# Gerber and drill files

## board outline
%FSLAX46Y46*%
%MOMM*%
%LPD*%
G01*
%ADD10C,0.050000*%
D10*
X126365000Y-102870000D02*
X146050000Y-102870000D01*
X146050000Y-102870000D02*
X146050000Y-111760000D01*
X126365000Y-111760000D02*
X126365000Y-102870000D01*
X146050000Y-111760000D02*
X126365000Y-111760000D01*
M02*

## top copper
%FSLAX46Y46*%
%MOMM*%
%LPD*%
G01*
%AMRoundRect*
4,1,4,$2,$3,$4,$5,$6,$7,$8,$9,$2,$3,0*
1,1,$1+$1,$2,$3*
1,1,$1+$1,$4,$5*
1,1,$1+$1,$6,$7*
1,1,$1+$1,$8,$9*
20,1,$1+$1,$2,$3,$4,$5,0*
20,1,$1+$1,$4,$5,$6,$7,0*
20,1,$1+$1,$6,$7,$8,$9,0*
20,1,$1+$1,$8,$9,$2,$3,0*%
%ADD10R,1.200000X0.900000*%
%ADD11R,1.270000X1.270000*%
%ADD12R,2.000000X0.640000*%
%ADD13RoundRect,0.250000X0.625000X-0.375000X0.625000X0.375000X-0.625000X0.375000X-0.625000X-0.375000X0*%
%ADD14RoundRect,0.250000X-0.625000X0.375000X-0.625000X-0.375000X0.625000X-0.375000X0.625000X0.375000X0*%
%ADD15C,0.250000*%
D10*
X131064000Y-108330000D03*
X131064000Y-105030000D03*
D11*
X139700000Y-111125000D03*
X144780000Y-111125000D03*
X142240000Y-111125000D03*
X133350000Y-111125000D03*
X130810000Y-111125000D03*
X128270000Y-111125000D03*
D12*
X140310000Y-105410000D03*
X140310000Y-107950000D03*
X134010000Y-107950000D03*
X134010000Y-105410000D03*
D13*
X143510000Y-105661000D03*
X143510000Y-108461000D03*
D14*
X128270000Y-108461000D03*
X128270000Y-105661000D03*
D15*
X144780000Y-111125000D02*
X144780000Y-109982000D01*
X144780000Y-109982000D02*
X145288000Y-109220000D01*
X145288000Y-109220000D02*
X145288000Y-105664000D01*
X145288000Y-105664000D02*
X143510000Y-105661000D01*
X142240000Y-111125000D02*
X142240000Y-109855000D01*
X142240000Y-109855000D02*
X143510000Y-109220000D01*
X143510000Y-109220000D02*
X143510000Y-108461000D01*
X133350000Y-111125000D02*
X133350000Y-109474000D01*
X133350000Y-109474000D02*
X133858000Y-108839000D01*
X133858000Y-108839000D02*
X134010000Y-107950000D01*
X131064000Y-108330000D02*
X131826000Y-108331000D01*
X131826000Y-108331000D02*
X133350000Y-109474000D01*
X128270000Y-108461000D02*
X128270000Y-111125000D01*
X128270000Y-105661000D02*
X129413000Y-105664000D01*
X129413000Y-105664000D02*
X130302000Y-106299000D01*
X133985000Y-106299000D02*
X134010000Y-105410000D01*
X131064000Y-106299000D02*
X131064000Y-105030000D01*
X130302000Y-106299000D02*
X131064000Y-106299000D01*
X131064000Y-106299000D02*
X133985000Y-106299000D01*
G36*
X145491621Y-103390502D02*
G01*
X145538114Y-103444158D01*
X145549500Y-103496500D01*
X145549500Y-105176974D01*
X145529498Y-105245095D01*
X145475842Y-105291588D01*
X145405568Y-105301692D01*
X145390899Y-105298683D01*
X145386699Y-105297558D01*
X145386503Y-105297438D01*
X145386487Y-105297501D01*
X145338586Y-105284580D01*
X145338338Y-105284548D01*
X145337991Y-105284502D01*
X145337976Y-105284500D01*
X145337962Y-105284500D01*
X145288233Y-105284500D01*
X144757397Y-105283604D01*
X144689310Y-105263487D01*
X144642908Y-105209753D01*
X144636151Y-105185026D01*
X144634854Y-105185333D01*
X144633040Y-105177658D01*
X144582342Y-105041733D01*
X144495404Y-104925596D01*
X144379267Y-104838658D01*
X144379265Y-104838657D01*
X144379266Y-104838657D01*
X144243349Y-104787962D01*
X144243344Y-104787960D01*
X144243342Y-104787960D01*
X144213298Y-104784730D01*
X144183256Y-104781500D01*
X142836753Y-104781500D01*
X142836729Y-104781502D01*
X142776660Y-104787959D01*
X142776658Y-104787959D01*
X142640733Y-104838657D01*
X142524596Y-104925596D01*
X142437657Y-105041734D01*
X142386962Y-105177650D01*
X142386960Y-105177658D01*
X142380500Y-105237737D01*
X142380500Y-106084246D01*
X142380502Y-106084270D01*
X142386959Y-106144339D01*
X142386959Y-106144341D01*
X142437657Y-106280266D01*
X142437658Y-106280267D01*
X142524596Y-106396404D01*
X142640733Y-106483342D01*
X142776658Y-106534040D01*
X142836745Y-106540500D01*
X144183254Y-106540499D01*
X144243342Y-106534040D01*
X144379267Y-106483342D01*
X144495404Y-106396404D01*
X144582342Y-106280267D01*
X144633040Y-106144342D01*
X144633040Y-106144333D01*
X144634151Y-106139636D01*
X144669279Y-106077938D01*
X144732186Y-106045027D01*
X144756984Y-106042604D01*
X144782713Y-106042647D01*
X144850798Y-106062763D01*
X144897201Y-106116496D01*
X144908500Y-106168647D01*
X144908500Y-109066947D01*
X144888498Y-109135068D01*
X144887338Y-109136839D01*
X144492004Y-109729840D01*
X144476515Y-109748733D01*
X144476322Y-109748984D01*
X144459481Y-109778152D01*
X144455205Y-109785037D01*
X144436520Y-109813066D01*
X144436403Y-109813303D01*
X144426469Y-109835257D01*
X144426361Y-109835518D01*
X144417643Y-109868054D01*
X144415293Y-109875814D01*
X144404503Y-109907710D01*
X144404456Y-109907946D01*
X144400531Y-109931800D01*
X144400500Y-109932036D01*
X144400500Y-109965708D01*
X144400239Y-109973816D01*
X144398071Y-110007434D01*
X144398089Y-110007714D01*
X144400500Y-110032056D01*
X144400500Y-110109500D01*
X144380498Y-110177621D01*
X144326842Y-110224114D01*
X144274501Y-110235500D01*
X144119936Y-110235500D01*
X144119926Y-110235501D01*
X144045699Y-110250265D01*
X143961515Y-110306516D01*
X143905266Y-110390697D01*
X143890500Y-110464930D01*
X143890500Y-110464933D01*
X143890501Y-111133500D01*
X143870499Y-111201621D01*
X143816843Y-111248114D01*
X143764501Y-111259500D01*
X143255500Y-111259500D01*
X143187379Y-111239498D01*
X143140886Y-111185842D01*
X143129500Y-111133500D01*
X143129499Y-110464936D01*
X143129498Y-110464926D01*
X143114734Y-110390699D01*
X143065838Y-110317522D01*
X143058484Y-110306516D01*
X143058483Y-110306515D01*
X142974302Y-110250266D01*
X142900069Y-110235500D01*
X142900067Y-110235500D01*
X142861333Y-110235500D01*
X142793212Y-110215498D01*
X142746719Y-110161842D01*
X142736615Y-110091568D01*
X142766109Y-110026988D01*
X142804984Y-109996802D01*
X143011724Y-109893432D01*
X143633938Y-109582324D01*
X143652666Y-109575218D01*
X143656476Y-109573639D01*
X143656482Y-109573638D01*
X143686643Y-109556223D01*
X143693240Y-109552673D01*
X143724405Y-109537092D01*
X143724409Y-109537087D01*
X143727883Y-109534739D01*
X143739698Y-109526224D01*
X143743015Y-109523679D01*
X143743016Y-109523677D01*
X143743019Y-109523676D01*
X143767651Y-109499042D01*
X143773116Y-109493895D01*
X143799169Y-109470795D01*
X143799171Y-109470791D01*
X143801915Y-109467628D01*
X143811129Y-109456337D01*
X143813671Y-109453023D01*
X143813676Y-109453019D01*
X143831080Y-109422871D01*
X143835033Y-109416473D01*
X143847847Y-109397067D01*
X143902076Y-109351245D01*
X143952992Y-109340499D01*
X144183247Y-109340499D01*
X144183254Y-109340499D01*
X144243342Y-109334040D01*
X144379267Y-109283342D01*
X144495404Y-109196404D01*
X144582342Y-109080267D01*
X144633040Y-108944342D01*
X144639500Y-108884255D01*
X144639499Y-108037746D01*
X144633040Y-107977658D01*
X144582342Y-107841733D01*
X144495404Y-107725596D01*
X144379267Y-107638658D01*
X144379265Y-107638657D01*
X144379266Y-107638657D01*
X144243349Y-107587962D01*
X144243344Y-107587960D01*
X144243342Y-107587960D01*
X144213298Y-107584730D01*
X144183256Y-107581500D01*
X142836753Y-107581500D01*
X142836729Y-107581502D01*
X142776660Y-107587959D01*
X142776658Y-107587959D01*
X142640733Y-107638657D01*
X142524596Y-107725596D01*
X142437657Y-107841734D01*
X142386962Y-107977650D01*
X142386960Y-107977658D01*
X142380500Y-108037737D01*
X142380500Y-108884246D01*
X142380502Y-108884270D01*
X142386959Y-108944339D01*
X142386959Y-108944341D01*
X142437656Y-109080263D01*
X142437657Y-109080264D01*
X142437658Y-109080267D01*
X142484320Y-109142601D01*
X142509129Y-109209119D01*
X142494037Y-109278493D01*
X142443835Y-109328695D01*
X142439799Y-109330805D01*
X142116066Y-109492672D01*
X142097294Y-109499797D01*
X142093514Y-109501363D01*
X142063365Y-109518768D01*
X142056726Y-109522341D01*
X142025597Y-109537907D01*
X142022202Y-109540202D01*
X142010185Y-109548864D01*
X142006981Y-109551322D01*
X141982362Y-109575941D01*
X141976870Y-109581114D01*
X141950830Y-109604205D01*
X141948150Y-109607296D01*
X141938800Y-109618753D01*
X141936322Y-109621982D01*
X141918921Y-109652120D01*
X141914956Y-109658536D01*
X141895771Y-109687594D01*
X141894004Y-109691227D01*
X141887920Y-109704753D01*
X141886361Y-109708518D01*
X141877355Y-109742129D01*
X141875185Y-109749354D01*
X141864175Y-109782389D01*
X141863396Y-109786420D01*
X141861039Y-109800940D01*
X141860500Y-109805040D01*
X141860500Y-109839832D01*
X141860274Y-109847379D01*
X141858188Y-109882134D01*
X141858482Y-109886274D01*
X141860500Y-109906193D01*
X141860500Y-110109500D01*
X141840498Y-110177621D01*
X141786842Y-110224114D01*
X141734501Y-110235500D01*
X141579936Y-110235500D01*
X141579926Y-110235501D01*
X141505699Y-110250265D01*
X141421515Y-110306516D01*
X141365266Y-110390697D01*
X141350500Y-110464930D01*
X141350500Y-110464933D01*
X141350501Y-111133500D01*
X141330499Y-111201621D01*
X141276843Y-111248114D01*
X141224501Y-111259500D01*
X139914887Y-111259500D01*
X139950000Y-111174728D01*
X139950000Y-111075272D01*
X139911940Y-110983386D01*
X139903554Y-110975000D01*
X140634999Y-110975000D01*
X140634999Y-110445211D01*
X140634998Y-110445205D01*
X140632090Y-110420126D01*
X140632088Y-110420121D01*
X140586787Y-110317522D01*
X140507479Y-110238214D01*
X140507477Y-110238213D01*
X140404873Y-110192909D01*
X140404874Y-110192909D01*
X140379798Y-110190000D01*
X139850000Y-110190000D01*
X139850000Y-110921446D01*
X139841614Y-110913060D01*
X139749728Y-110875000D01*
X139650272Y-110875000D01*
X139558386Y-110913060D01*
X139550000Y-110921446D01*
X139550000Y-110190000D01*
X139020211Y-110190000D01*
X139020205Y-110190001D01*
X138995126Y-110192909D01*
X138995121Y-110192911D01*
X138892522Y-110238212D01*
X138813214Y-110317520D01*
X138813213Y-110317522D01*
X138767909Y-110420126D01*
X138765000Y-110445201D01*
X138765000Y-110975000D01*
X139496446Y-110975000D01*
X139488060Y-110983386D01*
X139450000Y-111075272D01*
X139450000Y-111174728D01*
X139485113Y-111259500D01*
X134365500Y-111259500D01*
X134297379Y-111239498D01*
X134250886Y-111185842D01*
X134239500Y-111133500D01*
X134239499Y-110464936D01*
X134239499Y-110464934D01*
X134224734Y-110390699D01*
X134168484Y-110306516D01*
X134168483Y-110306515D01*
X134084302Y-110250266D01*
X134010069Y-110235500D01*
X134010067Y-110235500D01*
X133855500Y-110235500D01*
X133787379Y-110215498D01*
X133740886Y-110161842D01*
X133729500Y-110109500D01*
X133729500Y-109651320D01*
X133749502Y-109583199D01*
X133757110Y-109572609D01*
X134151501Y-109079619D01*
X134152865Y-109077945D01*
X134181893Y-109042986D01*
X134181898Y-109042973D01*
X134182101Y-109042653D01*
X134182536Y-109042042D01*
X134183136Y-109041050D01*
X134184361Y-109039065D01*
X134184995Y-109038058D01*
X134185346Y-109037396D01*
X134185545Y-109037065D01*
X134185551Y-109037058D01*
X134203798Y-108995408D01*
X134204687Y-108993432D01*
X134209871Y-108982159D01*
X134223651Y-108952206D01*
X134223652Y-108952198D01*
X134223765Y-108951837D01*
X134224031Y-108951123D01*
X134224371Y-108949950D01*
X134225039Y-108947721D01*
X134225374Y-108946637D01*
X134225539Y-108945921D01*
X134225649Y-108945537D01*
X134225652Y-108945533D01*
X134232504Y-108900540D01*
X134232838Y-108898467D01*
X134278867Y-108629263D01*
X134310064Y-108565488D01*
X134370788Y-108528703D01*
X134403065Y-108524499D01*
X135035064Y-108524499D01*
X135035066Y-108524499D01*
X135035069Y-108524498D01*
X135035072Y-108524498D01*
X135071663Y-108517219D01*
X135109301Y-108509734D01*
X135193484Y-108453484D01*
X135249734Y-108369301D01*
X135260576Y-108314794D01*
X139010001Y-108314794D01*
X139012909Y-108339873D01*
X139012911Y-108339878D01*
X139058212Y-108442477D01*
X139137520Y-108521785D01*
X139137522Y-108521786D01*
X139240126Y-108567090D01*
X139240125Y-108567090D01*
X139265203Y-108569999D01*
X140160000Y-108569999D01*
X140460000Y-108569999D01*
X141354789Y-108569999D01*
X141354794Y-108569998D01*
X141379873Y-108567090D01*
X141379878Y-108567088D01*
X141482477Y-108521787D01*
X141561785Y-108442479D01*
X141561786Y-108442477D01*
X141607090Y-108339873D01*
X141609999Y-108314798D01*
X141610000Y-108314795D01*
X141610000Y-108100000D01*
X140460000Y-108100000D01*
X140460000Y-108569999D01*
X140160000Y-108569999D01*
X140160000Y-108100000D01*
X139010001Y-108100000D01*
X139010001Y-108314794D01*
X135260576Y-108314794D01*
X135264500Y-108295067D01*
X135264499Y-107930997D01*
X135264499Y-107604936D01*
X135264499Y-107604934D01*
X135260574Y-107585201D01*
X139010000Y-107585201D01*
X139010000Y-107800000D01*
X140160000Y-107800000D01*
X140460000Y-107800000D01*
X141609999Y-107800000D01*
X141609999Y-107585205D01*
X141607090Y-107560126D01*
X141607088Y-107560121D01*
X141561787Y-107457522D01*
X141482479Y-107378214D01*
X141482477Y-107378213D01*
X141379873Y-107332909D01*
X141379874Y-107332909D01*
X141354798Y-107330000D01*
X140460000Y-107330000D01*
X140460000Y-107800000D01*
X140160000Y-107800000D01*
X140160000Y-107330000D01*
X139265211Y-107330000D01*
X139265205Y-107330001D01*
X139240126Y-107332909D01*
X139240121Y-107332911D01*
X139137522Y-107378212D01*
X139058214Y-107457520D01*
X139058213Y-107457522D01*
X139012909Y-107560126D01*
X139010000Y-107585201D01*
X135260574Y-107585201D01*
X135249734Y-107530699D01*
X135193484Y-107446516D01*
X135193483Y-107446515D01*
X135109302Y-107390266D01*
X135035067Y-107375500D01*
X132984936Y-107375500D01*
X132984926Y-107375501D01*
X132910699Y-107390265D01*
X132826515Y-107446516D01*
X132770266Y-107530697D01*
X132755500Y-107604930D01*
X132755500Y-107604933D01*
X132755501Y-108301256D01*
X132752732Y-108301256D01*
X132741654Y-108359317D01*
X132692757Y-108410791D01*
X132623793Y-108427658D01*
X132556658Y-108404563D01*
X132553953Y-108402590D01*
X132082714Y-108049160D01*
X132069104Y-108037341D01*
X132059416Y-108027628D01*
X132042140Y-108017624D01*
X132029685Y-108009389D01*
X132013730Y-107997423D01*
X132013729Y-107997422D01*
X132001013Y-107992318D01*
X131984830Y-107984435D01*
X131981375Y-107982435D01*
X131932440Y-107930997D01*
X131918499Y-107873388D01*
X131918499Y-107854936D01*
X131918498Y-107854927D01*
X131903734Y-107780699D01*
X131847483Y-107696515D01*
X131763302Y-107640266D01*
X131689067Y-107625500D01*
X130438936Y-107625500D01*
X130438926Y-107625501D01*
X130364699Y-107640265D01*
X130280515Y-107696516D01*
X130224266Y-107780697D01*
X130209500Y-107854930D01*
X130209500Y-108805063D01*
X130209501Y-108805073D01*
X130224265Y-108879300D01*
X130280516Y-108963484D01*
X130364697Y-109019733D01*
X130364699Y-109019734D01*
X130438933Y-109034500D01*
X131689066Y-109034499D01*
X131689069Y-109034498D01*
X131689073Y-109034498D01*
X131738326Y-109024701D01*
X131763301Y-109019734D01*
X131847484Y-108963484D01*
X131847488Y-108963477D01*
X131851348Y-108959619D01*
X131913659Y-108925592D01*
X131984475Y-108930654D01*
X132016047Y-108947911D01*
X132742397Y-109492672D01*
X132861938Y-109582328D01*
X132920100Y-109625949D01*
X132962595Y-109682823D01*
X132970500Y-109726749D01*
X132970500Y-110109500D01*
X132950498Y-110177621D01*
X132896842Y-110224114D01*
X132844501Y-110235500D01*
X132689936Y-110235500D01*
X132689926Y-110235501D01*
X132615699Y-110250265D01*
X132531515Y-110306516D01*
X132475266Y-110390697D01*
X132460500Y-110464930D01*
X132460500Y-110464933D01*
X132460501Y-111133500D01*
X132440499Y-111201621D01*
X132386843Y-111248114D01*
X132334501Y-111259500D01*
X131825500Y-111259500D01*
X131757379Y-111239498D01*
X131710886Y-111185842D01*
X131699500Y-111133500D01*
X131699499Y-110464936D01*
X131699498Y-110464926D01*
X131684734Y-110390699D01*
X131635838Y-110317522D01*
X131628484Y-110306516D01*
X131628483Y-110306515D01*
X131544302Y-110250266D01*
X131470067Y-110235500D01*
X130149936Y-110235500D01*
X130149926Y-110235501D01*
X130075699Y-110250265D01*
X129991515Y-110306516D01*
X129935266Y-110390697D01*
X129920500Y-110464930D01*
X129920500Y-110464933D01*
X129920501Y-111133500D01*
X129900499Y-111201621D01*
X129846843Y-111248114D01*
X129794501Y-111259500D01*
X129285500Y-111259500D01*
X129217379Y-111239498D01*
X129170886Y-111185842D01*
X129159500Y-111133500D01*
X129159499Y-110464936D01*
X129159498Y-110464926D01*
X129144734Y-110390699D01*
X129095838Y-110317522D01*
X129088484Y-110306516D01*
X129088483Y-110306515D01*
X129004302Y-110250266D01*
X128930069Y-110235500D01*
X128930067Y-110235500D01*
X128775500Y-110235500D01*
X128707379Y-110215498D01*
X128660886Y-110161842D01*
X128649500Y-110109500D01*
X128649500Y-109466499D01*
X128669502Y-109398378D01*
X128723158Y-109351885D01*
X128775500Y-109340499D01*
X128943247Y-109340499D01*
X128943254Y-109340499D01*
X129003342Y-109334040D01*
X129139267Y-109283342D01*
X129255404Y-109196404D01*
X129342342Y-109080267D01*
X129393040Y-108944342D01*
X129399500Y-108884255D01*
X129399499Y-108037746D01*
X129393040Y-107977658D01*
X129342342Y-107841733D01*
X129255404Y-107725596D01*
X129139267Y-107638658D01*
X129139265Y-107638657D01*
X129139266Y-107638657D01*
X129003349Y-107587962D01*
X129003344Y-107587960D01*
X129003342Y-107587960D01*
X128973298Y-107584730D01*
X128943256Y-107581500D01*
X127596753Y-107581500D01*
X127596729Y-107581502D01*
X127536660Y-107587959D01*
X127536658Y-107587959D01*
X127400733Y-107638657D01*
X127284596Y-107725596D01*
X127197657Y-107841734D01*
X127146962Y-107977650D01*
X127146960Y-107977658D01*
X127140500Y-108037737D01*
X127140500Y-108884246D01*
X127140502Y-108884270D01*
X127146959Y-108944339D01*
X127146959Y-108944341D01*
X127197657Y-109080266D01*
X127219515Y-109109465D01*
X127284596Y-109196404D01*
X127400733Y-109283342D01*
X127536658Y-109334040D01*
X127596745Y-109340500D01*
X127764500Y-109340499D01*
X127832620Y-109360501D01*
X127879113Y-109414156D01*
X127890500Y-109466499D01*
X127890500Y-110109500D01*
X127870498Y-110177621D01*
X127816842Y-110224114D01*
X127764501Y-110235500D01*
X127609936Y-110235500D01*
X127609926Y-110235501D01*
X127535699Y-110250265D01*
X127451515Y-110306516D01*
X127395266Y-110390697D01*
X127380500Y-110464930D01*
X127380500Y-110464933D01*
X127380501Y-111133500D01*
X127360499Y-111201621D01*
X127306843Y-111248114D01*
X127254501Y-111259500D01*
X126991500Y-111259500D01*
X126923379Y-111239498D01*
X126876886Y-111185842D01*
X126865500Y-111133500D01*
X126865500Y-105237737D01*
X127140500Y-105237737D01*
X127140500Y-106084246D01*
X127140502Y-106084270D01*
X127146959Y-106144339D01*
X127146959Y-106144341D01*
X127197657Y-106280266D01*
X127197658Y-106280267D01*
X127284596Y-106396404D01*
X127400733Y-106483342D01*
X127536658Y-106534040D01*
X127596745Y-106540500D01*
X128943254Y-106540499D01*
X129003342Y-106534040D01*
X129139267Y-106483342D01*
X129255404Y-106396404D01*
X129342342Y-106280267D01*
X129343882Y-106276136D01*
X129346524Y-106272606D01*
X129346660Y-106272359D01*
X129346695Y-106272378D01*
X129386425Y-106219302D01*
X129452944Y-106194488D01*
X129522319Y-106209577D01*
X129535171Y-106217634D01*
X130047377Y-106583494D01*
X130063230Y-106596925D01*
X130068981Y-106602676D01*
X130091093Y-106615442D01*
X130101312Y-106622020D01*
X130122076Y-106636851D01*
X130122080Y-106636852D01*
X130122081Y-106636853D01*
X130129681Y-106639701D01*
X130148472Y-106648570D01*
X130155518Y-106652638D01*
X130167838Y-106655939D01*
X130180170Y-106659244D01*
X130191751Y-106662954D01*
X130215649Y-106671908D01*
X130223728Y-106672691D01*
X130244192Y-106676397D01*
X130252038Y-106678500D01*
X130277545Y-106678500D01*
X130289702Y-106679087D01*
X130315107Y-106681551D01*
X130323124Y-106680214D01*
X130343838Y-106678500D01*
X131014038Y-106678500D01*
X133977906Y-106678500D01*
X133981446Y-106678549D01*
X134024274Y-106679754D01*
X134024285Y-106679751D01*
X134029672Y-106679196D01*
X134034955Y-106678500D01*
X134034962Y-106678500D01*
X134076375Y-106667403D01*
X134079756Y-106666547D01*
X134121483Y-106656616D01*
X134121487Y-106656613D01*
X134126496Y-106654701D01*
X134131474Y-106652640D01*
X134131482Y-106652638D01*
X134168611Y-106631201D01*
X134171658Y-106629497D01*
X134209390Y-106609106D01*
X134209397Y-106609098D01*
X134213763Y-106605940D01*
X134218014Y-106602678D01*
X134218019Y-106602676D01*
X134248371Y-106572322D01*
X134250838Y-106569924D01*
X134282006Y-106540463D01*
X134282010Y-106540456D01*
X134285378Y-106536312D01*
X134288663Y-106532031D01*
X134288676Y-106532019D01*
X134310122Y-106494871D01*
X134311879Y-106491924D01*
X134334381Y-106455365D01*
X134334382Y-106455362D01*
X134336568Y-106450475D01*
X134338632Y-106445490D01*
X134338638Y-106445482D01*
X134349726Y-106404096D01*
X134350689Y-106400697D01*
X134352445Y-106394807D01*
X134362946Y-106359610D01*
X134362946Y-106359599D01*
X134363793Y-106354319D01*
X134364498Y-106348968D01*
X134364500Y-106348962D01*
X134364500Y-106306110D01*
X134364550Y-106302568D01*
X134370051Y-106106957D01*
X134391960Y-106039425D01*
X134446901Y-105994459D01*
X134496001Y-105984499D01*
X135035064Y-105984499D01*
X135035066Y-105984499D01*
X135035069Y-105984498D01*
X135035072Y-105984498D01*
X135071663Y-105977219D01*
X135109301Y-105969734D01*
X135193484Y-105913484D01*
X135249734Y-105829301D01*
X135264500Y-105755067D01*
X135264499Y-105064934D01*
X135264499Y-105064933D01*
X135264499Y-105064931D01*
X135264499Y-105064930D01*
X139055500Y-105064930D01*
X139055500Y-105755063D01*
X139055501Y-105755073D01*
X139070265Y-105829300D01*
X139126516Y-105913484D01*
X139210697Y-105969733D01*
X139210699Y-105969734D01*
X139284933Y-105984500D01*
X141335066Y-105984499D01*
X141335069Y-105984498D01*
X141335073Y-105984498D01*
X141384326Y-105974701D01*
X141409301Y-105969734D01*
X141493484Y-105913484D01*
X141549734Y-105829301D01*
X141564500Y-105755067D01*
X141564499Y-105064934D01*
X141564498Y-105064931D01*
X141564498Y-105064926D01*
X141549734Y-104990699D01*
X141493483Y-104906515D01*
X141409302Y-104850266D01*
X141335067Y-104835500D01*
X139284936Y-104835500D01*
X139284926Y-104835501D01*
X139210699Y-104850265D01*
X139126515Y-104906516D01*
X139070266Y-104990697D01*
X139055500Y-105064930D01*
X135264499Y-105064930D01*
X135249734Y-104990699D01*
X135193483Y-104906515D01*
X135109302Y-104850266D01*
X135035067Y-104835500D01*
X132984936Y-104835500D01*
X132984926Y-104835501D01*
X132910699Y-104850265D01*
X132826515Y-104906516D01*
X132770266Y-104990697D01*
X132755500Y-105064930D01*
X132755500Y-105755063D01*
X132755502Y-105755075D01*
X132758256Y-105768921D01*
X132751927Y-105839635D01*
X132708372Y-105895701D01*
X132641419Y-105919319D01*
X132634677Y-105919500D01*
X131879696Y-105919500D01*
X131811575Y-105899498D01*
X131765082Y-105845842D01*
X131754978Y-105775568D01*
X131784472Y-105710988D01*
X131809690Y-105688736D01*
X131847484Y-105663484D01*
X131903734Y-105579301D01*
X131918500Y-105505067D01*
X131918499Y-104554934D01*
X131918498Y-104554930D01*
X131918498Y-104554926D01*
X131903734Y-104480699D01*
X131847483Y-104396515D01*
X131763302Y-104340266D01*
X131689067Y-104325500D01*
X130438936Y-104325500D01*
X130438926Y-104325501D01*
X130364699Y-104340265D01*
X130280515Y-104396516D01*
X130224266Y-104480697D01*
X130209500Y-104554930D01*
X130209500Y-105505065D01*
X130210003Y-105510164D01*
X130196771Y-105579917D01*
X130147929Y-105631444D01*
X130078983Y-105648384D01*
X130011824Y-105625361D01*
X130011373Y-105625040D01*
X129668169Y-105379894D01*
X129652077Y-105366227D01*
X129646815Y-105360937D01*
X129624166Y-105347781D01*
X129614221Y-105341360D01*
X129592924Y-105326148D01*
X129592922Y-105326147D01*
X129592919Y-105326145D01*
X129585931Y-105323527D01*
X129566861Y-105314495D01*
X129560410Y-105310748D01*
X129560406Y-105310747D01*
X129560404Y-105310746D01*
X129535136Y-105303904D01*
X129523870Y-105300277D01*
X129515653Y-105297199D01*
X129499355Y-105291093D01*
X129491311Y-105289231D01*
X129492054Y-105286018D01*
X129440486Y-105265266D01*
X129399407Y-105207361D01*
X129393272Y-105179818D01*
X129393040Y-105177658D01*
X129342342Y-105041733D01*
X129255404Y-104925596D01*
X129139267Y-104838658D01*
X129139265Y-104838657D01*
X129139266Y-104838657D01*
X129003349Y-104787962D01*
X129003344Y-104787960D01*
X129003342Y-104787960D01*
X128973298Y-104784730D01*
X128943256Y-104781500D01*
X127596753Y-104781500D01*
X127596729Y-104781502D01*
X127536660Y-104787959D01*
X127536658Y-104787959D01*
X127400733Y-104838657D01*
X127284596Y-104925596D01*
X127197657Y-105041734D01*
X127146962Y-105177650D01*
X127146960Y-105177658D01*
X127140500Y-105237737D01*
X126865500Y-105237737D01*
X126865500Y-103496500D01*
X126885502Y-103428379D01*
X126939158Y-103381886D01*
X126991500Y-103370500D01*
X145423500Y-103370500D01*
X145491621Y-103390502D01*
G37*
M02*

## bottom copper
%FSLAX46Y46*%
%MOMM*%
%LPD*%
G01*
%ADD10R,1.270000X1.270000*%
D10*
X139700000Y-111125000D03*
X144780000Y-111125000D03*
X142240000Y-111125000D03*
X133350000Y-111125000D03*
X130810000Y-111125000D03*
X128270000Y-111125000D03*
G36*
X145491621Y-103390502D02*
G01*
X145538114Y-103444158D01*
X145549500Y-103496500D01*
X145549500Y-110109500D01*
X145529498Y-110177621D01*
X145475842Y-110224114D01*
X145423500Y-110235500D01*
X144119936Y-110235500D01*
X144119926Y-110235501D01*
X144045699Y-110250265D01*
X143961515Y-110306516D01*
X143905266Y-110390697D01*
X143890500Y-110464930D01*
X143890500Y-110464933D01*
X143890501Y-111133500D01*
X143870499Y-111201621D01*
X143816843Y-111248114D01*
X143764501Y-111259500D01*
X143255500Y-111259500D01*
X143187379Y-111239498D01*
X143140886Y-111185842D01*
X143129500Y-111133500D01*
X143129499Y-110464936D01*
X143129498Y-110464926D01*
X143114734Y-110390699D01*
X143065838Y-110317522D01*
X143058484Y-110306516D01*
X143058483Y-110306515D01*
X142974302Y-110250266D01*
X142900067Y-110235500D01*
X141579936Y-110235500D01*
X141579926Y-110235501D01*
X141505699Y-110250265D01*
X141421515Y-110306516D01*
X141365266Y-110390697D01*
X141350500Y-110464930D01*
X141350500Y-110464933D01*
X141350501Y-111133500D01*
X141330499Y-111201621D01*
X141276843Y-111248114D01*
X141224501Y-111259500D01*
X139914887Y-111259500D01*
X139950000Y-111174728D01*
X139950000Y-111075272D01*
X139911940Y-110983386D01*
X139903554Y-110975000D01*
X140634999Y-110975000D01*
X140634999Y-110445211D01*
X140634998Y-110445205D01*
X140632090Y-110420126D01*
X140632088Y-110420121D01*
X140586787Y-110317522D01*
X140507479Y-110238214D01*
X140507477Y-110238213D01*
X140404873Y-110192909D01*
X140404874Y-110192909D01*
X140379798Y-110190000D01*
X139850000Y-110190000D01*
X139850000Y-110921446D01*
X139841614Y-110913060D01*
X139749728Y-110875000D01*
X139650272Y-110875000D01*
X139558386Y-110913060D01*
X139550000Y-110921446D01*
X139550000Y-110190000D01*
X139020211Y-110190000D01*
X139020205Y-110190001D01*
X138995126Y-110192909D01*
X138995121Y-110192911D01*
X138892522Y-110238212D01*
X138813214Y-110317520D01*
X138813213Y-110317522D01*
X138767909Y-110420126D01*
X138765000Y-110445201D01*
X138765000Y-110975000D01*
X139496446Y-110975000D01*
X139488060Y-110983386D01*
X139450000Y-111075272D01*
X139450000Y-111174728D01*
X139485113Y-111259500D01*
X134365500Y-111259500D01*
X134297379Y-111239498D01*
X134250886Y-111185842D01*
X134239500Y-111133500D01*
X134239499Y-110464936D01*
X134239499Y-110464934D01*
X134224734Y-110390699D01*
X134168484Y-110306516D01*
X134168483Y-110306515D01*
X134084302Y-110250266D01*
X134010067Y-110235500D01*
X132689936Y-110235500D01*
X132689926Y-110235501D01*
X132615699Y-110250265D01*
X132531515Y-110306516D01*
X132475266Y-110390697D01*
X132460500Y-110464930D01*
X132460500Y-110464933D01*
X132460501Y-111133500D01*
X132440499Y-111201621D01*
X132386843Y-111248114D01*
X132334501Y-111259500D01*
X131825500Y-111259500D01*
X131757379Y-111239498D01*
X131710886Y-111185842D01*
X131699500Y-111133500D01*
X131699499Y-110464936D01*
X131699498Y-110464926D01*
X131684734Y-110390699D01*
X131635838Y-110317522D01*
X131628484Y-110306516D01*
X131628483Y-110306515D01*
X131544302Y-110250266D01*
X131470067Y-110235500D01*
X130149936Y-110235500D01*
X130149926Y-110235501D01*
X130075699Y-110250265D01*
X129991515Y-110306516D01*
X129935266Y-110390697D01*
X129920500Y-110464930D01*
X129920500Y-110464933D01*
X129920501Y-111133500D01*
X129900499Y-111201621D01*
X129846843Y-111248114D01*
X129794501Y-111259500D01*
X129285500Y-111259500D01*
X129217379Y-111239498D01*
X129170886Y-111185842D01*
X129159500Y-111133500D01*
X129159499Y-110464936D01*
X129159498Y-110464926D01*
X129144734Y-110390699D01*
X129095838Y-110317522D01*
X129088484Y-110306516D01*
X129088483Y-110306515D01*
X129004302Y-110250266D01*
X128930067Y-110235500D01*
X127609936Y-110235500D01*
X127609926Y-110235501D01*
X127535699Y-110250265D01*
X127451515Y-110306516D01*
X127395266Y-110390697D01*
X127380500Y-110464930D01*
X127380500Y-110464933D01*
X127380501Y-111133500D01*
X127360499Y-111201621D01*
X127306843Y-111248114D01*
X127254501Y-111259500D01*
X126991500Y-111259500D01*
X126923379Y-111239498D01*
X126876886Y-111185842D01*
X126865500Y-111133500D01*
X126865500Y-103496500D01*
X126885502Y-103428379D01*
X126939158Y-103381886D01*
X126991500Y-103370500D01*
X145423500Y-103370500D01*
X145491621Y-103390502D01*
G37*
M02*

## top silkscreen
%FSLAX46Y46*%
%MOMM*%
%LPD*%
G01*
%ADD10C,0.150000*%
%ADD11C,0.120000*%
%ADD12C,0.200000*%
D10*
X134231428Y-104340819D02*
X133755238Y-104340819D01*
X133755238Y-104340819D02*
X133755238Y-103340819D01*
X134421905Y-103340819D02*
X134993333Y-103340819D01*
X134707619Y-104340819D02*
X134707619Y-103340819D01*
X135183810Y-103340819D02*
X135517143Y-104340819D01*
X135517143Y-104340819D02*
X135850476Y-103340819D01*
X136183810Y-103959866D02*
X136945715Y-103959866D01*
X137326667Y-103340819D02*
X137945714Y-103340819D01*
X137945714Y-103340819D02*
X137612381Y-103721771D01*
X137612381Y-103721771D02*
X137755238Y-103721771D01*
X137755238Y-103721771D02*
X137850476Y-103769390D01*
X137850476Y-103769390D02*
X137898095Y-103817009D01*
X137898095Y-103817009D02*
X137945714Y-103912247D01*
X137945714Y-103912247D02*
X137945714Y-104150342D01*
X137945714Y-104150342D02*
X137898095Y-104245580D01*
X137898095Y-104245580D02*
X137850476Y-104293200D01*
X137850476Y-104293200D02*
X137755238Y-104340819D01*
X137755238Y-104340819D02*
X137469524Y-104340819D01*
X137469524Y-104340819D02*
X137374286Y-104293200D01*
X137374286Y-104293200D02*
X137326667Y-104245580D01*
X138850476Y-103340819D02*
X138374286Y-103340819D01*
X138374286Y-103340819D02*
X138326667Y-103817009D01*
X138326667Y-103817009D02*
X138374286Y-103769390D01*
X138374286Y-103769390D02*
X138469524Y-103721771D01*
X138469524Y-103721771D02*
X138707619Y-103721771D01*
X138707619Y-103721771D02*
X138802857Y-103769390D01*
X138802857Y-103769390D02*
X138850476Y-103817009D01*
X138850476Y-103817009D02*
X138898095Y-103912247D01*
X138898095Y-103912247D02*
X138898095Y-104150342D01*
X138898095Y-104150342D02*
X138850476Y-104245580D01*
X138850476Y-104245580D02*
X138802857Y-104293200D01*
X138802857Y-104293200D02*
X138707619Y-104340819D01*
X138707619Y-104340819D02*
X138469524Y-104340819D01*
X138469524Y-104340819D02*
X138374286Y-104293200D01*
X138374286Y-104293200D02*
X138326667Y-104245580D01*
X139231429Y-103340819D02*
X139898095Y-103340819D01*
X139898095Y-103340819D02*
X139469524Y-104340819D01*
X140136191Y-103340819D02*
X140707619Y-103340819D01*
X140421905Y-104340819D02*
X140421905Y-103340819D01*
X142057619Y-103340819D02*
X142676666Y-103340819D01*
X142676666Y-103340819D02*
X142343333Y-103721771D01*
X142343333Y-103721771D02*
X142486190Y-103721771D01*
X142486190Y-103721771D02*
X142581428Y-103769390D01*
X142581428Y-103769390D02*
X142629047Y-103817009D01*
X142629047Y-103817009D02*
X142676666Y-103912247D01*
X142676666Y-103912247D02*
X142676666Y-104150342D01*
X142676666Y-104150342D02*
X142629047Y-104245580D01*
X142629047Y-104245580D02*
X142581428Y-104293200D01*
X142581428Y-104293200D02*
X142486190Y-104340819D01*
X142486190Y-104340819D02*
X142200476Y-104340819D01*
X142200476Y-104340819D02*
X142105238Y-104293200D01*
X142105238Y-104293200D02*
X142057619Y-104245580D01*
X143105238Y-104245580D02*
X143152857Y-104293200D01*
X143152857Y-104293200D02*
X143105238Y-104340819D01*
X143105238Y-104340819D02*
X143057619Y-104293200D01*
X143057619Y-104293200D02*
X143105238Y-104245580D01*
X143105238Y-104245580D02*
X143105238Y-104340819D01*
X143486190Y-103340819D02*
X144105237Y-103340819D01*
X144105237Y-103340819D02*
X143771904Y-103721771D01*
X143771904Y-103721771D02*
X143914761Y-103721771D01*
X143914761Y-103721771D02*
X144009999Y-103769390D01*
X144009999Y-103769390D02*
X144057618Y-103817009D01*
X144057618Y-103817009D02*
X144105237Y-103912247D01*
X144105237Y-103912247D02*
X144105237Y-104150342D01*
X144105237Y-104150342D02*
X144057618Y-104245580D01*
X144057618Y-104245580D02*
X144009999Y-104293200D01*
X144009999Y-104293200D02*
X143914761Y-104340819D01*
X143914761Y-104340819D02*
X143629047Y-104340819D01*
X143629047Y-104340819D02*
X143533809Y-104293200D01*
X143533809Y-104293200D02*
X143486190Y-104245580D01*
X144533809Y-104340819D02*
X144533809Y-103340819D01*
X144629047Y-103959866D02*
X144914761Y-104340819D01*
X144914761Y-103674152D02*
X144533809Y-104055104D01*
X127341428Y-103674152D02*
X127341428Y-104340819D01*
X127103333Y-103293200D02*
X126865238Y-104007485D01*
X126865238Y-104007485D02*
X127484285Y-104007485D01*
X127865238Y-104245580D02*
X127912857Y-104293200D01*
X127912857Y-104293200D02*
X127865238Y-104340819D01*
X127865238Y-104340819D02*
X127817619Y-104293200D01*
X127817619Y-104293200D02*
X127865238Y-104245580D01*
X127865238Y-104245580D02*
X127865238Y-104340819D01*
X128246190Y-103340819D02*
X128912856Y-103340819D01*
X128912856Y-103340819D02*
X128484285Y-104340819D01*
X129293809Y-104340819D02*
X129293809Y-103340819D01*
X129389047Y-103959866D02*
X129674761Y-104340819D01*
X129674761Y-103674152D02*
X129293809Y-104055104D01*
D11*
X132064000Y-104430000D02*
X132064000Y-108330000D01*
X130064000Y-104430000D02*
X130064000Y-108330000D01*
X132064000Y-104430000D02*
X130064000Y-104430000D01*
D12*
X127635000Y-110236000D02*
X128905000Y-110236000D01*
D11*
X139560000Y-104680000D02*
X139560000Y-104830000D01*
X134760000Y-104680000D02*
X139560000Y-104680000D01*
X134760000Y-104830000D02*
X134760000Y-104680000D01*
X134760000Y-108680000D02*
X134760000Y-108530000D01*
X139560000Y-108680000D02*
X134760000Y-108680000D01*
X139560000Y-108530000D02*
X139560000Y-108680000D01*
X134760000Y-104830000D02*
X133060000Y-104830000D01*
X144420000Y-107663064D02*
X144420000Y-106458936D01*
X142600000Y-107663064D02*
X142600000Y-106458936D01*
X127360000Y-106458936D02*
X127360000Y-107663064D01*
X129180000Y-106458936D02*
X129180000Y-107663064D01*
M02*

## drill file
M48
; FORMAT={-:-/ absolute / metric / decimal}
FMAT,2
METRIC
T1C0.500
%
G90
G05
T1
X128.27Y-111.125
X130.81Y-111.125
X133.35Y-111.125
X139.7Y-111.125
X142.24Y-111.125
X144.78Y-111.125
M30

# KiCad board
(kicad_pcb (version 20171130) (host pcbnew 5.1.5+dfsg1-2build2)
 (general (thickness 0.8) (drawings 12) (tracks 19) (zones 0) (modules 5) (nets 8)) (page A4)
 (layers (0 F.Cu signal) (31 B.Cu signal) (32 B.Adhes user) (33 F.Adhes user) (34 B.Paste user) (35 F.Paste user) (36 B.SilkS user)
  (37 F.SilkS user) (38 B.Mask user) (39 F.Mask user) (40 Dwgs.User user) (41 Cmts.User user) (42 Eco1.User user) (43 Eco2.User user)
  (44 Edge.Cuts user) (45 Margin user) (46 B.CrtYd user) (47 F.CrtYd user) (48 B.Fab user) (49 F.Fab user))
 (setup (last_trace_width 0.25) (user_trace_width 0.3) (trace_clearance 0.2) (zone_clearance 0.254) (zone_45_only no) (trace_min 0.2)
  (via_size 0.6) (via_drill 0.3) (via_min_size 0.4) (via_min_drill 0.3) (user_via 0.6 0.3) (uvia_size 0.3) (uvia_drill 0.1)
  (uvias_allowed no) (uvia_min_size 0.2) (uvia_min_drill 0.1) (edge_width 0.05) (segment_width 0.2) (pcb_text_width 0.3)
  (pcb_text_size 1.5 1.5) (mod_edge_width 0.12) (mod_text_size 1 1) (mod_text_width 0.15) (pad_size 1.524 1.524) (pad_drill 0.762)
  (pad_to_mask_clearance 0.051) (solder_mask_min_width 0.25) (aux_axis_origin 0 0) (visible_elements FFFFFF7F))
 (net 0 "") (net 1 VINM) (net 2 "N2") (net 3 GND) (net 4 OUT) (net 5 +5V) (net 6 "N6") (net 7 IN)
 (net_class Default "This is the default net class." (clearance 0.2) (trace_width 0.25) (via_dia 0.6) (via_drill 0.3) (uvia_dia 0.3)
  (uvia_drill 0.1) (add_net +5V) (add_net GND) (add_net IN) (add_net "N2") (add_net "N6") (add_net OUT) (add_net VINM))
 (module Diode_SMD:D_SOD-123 (layer F.Cu) (at 131.064 106.68 270)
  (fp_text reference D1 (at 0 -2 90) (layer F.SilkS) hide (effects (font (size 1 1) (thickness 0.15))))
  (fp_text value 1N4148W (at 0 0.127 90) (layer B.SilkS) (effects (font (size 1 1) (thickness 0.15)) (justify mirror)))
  (fp_line (start -2.25 -1) (end 1.65 -1) (layer F.SilkS) (width 0.12))
  (fp_line (start -2.25 1) (end 1.65 1) (layer F.SilkS) (width 0.12))
  (fp_line (start -2.25 -1) (end -2.25 1) (layer F.SilkS) (width 0.12))
  (pad 2 smd rect (at 1.65 0 270) (size 0.9 1.2) (layers F.Cu F.Paste F.Mask) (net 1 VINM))
  (pad 1 smd rect (at -1.65 0 270) (size 0.9 1.2) (layers F.Cu F.Paste F.Mask) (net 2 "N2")))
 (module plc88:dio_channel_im (layer F.Cu) (at 135.255 108.585)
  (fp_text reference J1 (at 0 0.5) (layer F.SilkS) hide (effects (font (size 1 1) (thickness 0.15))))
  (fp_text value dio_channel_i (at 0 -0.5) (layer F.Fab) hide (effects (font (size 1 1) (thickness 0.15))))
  (fp_line (start -7.62 1.651) (end -6.35 1.651) (layer F.SilkS) (width 0.2))
  (pad 4 thru_hole rect (at 4.445 2.54) (size 1.27 1.27) (drill 0.5) (layers *.Cu *.Mask) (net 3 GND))
  (pad 6 thru_hole rect (at 9.525 2.54) (size 1.27 1.27) (drill 0.5) (layers *.Cu *.Mask) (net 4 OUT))
  (pad 5 thru_hole rect (at 6.985 2.54) (size 1.27 1.27) (drill 0.5) (layers *.Cu *.Mask) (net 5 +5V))
  (pad 3 thru_hole rect (at -1.905 2.54) (size 1.27 1.27) (drill 0.5) (layers *.Cu *.Mask) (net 1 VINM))
  (pad 2 thru_hole rect (at -4.445 2.54) (size 1.27 1.27) (drill 0.5) (layers *.Cu *.Mask) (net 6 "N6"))
  (pad 1 thru_hole rect (at -6.985 2.54) (size 1.27 1.27) (drill 0.5) (layers *.Cu *.Mask) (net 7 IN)))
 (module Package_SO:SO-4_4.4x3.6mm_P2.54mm (layer F.Cu) (at 137.16 106.68)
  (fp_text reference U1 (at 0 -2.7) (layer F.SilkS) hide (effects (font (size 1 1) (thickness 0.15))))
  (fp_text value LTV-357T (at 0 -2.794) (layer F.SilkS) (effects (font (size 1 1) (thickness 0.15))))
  (fp_line (start 2.4 -2) (end 2.4 -1.85) (layer F.SilkS) (width 0.12))
  (fp_line (start -2.4 -2) (end 2.4 -2) (layer F.SilkS) (width 0.12))
  (fp_line (start -2.4 -1.85) (end -2.4 -2) (layer F.SilkS) (width 0.12))
  (fp_line (start -2.4 2) (end -2.4 1.85) (layer F.SilkS) (width 0.12))
  (fp_line (start 2.4 2) (end -2.4 2) (layer F.SilkS) (width 0.12))
  (fp_line (start 2.4 1.85) (end 2.4 2) (layer F.SilkS) (width 0.12))
  (fp_line (start -2.4 -1.85) (end -4.1 -1.85) (layer F.SilkS) (width 0.12))
  (pad 4 smd rect (at 3.15 -1.27) (size 2 0.64) (layers F.Cu F.Paste F.Mask) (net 4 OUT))
  (pad 3 smd rect (at 3.15 1.27) (size 2 0.64) (layers F.Cu F.Paste F.Mask) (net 3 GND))
  (pad 2 smd rect (at -3.15 1.27) (size 2 0.64) (layers F.Cu F.Paste F.Mask) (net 1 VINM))
  (pad 1 smd rect (at -3.15 -1.27) (size 2 0.64) (layers F.Cu F.Paste F.Mask) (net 2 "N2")))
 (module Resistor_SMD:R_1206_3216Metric (layer F.Cu) (at 143.51 107.061 90)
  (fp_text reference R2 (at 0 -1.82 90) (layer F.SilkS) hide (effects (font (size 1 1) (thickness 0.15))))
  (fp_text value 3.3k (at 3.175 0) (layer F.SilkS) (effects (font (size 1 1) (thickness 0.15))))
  (fp_line (start -0.602064 0.91) (end 0.602064 0.91) (layer F.SilkS) (width 0.12))
  (fp_line (start -0.602064 -0.91) (end 0.602064 -0.91) (layer F.SilkS) (width 0.12))
  (pad 2 smd roundrect (at 1.4 0 90) (size 1.25 1.75) (layers F.Cu F.Paste F.Mask) (roundrect_rratio 0.2) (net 4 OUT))
  (pad 1 smd roundrect (at -1.4 0 90) (size 1.25 1.75) (layers F.Cu F.Paste F.Mask) (roundrect_rratio 0.2) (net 5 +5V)))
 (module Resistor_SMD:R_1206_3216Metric (layer F.Cu) (at 128.27 107.061 270)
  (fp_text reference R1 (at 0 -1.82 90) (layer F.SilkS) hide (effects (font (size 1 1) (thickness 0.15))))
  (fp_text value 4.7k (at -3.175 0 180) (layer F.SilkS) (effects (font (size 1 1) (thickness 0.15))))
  (fp_line (start -0.602064 0.91) (end 0.602064 0.91) (layer F.SilkS) (width 0.12))
  (fp_line (start -0.602064 -0.91) (end 0.602064 -0.91) (layer F.SilkS) (width 0.12))
  (pad 2 smd roundrect (at 1.4 0 270) (size 1.25 1.75) (layers F.Cu F.Paste F.Mask) (roundrect_rratio 0.2) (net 7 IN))
  (pad 1 smd roundrect (at -1.4 0 270) (size 1.25 1.75) (layers F.Cu F.Paste F.Mask) (roundrect_rratio 0.2) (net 2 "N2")))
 (gr_line (start 126.365 102.87) (end 146.05 102.87) (layer Edge.Cuts) (width 0.05))
 (gr_line (start 146.05 102.87) (end 146.05 111.76) (layer Edge.Cuts) (width 0.05))
 (gr_line (start 126.365 111.76) (end 126.365 102.87) (layer Edge.Cuts) (width 0.05))
 (gr_line (start 146.05 111.76) (end 126.365 111.76) (layer Edge.Cuts) (width 0.05))
 (segment (start 144.78 111.125) (end 144.78 109.982) (width 0.25) (layer F.Cu) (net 4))
 (segment (start 144.78 109.982) (end 145.288 109.22) (width 0.25) (layer F.Cu) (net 4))
 (segment (start 145.288 109.22) (end 145.288 105.664) (width 0.25) (layer F.Cu) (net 4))
 (segment (start 145.288 105.664) (end 143.51 105.661) (width 0.25) (layer F.Cu) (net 4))
 (segment (start 142.24 111.125) (end 142.24 109.855) (width 0.25) (layer F.Cu) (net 5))
 (segment (start 142.24 109.855) (end 143.51 109.22) (width 0.25) (layer F.Cu) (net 5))
 (segment (start 143.51 109.22) (end 143.51 108.461) (width 0.25) (layer F.Cu) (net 5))
 (segment (start 133.35 111.125) (end 133.35 109.474) (width 0.25) (layer F.Cu) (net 1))
 (segment (start 133.35 109.474) (end 133.858 108.839) (width 0.25) (layer F.Cu) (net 1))
 (segment (start 133.858 108.839) (end 134.01 107.95) (width 0.25) (layer F.Cu) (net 1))
 (segment (start 131.064 108.33) (end 131.826 108.331) (width 0.25) (layer F.Cu) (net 1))
 (segment (start 131.826 108.331) (end 133.35 109.474) (width 0.25) (layer F.Cu) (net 1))
 (segment (start 128.27 108.461) (end 128.27 111.125) (width 0.25) (layer F.Cu) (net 7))
 (segment (start 128.27 105.661) (end 129.413 105.664) (width 0.25) (layer F.Cu) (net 2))
 (segment (start 129.413 105.664) (end 130.302 106.299) (width 0.25) (layer F.Cu) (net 2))
 (segment (start 133.985 106.299) (end 134.01 105.41) (width 0.25) (layer F.Cu) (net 2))
 (segment (start 131.064 106.299) (end 131.064 105.03) (width 0.25) (layer F.Cu) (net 2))
 (segment (start 130.302 106.299) (end 131.064 106.299) (width 0.25) (layer F.Cu) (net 2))
 (segment (start 131.064 106.299) (end 133.985 106.299) (width 0.25) (layer F.Cu) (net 2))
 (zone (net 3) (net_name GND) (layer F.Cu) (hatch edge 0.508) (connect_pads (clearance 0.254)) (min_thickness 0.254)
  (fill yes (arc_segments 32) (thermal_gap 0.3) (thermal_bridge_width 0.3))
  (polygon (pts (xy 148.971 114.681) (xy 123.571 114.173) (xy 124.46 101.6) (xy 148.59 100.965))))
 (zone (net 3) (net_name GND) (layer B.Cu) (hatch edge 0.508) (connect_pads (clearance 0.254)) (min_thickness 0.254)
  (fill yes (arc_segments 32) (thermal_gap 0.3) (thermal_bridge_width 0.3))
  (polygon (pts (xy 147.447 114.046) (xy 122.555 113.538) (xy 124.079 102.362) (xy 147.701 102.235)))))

